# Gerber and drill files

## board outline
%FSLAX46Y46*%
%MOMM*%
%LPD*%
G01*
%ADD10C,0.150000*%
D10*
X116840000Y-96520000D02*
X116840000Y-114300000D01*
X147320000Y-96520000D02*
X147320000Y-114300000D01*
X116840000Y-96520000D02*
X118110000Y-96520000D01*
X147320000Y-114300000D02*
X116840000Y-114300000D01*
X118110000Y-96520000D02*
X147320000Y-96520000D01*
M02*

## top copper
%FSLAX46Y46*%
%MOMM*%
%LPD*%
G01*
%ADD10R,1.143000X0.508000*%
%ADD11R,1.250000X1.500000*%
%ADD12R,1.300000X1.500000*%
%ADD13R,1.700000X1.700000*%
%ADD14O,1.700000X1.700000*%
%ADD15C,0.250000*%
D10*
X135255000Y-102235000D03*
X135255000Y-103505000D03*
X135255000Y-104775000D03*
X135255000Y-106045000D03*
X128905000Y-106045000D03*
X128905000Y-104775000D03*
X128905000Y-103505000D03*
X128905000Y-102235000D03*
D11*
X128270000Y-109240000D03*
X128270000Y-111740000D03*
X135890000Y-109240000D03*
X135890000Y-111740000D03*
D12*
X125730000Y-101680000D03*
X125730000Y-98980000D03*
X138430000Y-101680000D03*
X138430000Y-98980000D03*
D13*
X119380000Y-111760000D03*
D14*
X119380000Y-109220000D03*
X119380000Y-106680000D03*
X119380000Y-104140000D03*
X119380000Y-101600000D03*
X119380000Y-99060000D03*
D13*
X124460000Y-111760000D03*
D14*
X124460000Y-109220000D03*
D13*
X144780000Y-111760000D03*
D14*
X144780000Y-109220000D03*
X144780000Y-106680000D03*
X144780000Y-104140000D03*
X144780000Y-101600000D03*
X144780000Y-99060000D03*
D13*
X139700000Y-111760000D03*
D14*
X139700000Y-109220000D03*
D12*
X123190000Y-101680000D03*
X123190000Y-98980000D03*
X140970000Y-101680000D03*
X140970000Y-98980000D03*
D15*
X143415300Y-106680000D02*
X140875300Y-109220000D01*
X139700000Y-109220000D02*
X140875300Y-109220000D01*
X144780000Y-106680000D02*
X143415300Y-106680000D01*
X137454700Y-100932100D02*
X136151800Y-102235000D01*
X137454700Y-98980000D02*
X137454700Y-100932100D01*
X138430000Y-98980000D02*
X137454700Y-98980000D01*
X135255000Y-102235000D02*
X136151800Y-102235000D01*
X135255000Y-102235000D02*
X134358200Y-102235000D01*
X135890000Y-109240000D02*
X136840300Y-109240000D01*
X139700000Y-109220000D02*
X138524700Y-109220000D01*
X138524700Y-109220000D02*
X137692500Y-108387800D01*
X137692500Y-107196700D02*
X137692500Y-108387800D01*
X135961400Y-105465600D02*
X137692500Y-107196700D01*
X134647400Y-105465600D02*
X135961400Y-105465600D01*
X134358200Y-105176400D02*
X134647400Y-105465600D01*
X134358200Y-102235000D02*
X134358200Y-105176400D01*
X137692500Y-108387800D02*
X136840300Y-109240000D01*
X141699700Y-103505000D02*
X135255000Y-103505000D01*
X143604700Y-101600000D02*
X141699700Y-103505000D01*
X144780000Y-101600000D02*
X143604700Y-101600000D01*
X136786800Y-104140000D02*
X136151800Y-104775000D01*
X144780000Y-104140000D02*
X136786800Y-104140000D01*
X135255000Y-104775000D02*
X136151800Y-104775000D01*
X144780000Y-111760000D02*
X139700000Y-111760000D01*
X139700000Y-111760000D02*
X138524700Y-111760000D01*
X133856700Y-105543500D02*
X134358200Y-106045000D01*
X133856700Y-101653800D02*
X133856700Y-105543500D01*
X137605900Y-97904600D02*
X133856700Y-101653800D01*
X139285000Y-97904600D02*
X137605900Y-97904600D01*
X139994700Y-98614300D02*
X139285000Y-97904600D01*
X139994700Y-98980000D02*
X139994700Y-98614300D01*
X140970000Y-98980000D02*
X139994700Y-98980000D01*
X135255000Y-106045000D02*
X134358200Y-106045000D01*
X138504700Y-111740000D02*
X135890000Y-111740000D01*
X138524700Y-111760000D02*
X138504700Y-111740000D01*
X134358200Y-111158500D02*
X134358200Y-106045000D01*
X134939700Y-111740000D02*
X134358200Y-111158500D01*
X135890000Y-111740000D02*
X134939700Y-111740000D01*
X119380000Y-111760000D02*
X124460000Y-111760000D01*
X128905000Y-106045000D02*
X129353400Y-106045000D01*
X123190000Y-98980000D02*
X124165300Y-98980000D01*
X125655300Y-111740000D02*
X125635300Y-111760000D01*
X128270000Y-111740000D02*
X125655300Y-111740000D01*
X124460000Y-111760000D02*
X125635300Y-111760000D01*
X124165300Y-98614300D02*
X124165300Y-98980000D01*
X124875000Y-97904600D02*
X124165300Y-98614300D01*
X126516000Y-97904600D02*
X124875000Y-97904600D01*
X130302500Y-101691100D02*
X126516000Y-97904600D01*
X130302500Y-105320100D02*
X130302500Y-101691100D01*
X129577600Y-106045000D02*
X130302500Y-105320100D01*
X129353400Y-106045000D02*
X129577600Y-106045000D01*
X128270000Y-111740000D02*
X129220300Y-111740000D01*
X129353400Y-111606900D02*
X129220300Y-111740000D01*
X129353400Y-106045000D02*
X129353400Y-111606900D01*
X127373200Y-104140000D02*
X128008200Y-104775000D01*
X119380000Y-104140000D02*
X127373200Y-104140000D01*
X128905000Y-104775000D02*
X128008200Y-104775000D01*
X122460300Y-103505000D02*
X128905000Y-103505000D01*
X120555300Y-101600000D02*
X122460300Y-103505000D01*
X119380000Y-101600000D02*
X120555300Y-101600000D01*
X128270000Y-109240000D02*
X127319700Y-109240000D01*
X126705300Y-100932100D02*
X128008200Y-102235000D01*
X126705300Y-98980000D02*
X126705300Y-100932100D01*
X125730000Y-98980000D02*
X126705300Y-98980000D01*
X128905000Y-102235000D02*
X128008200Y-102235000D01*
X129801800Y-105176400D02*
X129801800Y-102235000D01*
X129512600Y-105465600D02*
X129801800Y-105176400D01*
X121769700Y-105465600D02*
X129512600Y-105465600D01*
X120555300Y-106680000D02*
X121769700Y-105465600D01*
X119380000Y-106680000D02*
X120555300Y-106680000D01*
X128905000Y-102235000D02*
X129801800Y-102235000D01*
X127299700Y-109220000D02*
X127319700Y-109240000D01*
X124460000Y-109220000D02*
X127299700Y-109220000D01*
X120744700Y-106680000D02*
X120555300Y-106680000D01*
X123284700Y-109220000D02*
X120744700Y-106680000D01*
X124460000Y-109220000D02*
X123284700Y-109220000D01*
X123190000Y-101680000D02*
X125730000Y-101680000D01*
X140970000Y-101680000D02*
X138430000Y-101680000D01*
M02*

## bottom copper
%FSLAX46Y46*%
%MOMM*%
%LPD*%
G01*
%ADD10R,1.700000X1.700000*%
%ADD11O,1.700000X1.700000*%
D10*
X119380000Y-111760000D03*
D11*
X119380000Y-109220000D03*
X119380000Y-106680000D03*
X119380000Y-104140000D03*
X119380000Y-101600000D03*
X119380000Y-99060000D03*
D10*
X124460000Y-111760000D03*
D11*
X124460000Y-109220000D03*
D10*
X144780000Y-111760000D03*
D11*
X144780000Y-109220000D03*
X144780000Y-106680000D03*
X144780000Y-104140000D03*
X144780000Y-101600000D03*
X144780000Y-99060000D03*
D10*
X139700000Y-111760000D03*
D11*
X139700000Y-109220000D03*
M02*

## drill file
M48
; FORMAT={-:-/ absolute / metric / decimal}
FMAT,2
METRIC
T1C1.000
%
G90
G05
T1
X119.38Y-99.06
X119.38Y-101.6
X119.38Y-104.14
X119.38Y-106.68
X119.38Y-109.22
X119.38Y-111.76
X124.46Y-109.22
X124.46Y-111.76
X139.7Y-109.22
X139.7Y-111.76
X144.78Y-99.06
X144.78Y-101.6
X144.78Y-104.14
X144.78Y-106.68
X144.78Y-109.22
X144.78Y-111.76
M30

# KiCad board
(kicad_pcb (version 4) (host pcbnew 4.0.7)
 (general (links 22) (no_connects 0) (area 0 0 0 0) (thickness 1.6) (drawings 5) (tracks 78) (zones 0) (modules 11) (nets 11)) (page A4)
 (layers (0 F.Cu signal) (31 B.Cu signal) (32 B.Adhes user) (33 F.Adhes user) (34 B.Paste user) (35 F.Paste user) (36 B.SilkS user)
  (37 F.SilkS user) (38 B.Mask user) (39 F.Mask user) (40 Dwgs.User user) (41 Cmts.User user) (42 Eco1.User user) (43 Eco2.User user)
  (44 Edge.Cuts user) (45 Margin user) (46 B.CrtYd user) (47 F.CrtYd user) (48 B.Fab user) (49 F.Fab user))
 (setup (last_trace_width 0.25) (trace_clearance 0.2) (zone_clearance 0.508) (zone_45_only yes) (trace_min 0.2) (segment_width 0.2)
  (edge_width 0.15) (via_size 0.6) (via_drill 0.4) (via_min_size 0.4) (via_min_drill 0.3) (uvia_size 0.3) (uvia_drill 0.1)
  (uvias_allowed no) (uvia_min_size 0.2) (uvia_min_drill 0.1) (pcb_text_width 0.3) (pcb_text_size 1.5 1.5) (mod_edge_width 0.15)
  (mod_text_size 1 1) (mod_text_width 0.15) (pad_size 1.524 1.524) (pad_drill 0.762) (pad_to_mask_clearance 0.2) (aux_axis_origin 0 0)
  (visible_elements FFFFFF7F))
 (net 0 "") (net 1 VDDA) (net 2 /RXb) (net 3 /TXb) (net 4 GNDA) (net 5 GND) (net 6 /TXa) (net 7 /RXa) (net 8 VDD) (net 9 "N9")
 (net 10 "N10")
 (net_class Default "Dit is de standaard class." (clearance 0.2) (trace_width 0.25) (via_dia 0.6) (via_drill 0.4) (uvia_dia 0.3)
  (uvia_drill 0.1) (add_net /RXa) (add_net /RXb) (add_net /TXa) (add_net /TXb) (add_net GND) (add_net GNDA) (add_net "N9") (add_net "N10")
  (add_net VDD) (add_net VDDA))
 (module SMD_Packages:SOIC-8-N (layer F.Cu) (at 132.08 104.14 270)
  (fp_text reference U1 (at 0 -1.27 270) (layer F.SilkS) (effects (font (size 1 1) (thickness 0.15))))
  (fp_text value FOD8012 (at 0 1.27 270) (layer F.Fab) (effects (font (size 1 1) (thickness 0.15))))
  (pad 8 smd rect (at -1.905 -3.175 270) (size 0.508 1.143) (layers F.Cu F.Paste F.Mask) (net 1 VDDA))
  (pad 7 smd rect (at -0.635 -3.175 270) (size 0.508 1.143) (layers F.Cu F.Paste F.Mask) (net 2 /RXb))
  (pad 6 smd rect (at 0.635 -3.175 270) (size 0.508 1.143) (layers F.Cu F.Paste F.Mask) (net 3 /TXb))
  (pad 5 smd rect (at 1.905 -3.175 270) (size 0.508 1.143) (layers F.Cu F.Paste F.Mask) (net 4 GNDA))
  (pad 4 smd rect (at 1.905 3.175 270) (size 0.508 1.143) (layers F.Cu F.Paste F.Mask) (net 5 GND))
  (pad 3 smd rect (at 0.635 3.175 270) (size 0.508 1.143) (layers F.Cu F.Paste F.Mask) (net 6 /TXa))
  (pad 2 smd rect (at -0.635 3.175 270) (size 0.508 1.143) (layers F.Cu F.Paste F.Mask) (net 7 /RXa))
  (pad 1 smd rect (at -1.905 3.175 270) (size 0.508 1.143) (layers F.Cu F.Paste F.Mask) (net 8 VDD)))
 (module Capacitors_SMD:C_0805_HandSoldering (layer F.Cu) (at 128.27 110.49 270)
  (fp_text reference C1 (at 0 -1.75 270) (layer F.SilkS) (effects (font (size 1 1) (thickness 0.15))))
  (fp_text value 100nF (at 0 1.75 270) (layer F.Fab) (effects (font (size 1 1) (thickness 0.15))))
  (pad 1 smd rect (at -1.25 0 270) (size 1.5 1.25) (layers F.Cu F.Paste F.Mask) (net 8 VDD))
  (pad 2 smd rect (at 1.25 0 270) (size 1.5 1.25) (layers F.Cu F.Paste F.Mask) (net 5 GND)))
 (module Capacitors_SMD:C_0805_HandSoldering (layer F.Cu) (at 135.89 110.49 270)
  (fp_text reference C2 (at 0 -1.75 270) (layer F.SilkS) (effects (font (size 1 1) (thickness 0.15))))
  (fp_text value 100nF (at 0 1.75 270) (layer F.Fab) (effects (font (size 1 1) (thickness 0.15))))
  (pad 1 smd rect (at -1.25 0 270) (size 1.5 1.25) (layers F.Cu F.Paste F.Mask) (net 1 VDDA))
  (pad 2 smd rect (at 1.25 0 270) (size 1.5 1.25) (layers F.Cu F.Paste F.Mask) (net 4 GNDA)))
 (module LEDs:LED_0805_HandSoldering (layer F.Cu) (at 125.73 100.33 90)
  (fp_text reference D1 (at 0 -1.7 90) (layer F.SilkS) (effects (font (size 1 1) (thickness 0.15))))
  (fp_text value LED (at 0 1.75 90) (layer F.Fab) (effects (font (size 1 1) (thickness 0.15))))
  (pad 1 smd rect (at -1.35 0 90) (size 1.5 1.3) (layers F.Cu F.Paste F.Mask) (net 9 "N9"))
  (pad 2 smd rect (at 1.35 0 90) (size 1.5 1.3) (layers F.Cu F.Paste F.Mask) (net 8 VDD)))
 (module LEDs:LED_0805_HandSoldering (layer F.Cu) (at 138.43 100.33 90)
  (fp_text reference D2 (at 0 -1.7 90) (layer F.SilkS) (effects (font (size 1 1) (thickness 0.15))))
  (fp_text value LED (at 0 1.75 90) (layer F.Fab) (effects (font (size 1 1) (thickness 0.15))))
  (pad 1 smd rect (at -1.35 0 90) (size 1.5 1.3) (layers F.Cu F.Paste F.Mask) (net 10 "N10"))
  (pad 2 smd rect (at 1.35 0 90) (size 1.5 1.3) (layers F.Cu F.Paste F.Mask) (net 1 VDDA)))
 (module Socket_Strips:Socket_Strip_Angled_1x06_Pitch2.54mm (layer B.Cu) (at 119.38 111.76)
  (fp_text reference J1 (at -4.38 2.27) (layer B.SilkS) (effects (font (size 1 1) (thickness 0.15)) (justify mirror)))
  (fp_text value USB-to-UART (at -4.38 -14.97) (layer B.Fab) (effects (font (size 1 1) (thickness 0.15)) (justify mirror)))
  (pad 1 thru_hole rect (at 0 0) (size 1.7 1.7) (drill 1) (layers *.Cu *.Mask) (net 5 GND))
  (pad 2 thru_hole oval (at 0 -2.54) (size 1.7 1.7) (drill 1) (layers *.Cu *.Mask))
  (pad 3 thru_hole oval (at 0 -5.08) (size 1.7 1.7) (drill 1) (layers *.Cu *.Mask) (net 8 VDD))
  (pad 4 thru_hole oval (at 0 -7.62) (size 1.7 1.7) (drill 1) (layers *.Cu *.Mask) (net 6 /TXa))
  (pad 5 thru_hole oval (at 0 -10.16) (size 1.7 1.7) (drill 1) (layers *.Cu *.Mask) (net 7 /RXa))
  (pad 6 thru_hole oval (at 0 -12.7) (size 1.7 1.7) (drill 1) (layers *.Cu *.Mask)))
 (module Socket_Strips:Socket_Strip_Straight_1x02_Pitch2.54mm (layer F.Cu) (at 124.46 111.76 180)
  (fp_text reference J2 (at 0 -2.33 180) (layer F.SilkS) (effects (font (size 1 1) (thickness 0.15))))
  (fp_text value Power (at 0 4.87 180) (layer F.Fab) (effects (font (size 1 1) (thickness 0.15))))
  (pad 1 thru_hole rect (at 0 0 180) (size 1.7 1.7) (drill 1) (layers *.Cu *.Mask) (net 5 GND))
  (pad 2 thru_hole oval (at 0 2.54 180) (size 1.7 1.7) (drill 1) (layers *.Cu *.Mask) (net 8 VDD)))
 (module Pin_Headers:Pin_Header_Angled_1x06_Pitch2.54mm (layer B.Cu) (at 144.78 111.76)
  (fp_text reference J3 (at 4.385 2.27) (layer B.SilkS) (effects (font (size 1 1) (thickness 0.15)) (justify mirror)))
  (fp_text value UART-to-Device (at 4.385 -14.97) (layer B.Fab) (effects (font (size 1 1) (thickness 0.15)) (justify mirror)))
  (pad 1 thru_hole rect (at 0 0) (size 1.7 1.7) (drill 1) (layers *.Cu *.Mask) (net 4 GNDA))
  (pad 2 thru_hole oval (at 0 -2.54) (size 1.7 1.7) (drill 1) (layers *.Cu *.Mask))
  (pad 3 thru_hole oval (at 0 -5.08) (size 1.7 1.7) (drill 1) (layers *.Cu *.Mask) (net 1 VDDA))
  (pad 4 thru_hole oval (at 0 -7.62) (size 1.7 1.7) (drill 1) (layers *.Cu *.Mask) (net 3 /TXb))
  (pad 5 thru_hole oval (at 0 -10.16) (size 1.7 1.7) (drill 1) (layers *.Cu *.Mask) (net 2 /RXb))
  (pad 6 thru_hole oval (at 0 -12.7) (size 1.7 1.7) (drill 1) (layers *.Cu *.Mask)))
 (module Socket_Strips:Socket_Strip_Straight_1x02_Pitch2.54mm (layer F.Cu) (at 139.7 111.76 180)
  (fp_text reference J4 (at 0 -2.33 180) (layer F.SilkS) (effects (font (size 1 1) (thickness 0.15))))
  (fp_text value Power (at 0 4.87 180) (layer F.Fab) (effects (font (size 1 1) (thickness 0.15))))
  (pad 1 thru_hole rect (at 0 0 180) (size 1.7 1.7) (drill 1) (layers *.Cu *.Mask) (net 4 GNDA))
  (pad 2 thru_hole oval (at 0 2.54 180) (size 1.7 1.7) (drill 1) (layers *.Cu *.Mask) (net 1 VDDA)))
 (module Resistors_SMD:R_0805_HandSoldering (layer F.Cu) (at 123.19 100.33 90)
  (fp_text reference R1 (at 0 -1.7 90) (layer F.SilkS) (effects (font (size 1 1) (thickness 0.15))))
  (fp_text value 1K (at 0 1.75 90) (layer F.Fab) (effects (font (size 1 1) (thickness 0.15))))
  (pad 1 smd rect (at -1.35 0 90) (size 1.5 1.3) (layers F.Cu F.Paste F.Mask) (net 9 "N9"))
  (pad 2 smd rect (at 1.35 0 90) (size 1.5 1.3) (layers F.Cu F.Paste F.Mask) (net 5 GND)))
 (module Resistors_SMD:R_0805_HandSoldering (layer F.Cu) (at 140.97 100.33 90)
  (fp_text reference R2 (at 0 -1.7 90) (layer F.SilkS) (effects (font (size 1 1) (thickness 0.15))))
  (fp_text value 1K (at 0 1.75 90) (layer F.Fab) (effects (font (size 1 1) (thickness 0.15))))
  (pad 1 smd rect (at -1.35 0 90) (size 1.5 1.3) (layers F.Cu F.Paste F.Mask) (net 10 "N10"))
  (pad 2 smd rect (at 1.35 0 90) (size 1.5 1.3) (layers F.Cu F.Paste F.Mask) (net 4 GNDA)))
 (gr_line (start 116.84 96.52) (end 116.84 114.3) (angle 90) (layer Edge.Cuts) (width 0.15))
 (gr_line (start 147.32 96.52) (end 147.32 114.3) (angle 90) (layer Edge.Cuts) (width 0.15))
 (gr_line (start 116.84 96.52) (end 118.11 96.52) (angle 90) (layer Edge.Cuts) (width 0.15))
 (gr_line (start 147.32 114.3) (end 116.84 114.3) (angle 90) (layer Edge.Cuts) (width 0.15))
 (gr_line (start 118.11 96.52) (end 147.32 96.52) (angle 90) (layer Edge.Cuts) (width 0.15))
 (segment (start 143.4153 106.68) (end 140.8753 109.22) (width 0.25) (layer F.Cu) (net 1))
 (segment (start 139.7 109.22) (end 140.8753 109.22) (width 0.25) (layer F.Cu) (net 1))
 (segment (start 144.78 106.68) (end 143.4153 106.68) (width 0.25) (layer F.Cu) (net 1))
 (segment (start 137.4547 100.9321) (end 136.1518 102.235) (width 0.25) (layer F.Cu) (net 1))
 (segment (start 137.4547 98.98) (end 137.4547 100.9321) (width 0.25) (layer F.Cu) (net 1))
 (segment (start 138.43 98.98) (end 137.4547 98.98) (width 0.25) (layer F.Cu) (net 1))
 (segment (start 135.255 102.235) (end 136.1518 102.235) (width 0.25) (layer F.Cu) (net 1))
 (segment (start 135.255 102.235) (end 134.3582 102.235) (width 0.25) (layer F.Cu) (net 1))
 (segment (start 135.89 109.24) (end 136.8403 109.24) (width 0.25) (layer F.Cu) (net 1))
 (segment (start 139.7 109.22) (end 138.5247 109.22) (width 0.25) (layer F.Cu) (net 1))
 (segment (start 138.5247 109.22) (end 137.6925 108.3878) (width 0.25) (layer F.Cu) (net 1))
 (segment (start 137.6925 107.1967) (end 137.6925 108.3878) (width 0.25) (layer F.Cu) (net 1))
 (segment (start 135.9614 105.4656) (end 137.6925 107.1967) (width 0.25) (layer F.Cu) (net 1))
 (segment (start 134.6474 105.4656) (end 135.9614 105.4656) (width 0.25) (layer F.Cu) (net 1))
 (segment (start 134.3582 105.1764) (end 134.6474 105.4656) (width 0.25) (layer F.Cu) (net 1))
 (segment (start 134.3582 102.235) (end 134.3582 105.1764) (width 0.25) (layer F.Cu) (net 1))
 (segment (start 137.6925 108.3878) (end 136.8403 109.24) (width 0.25) (layer F.Cu) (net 1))
 (segment (start 141.6997 103.505) (end 135.255 103.505) (width 0.25) (layer F.Cu) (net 2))
 (segment (start 143.6047 101.6) (end 141.6997 103.505) (width 0.25) (layer F.Cu) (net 2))
 (segment (start 144.78 101.6) (end 143.6047 101.6) (width 0.25) (layer F.Cu) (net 2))
 (segment (start 136.7868 104.14) (end 136.1518 104.775) (width 0.25) (layer F.Cu) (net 3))
 (segment (start 144.78 104.14) (end 136.7868 104.14) (width 0.25) (layer F.Cu) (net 3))
 (segment (start 135.255 104.775) (end 136.1518 104.775) (width 0.25) (layer F.Cu) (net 3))
 (segment (start 144.78 111.76) (end 139.7 111.76) (width 0.25) (layer F.Cu) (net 4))
 (segment (start 139.7 111.76) (end 138.5247 111.76) (width 0.25) (layer F.Cu) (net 4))
 (segment (start 133.8567 105.5435) (end 134.3582 106.045) (width 0.25) (layer F.Cu) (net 4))
 (segment (start 133.8567 101.6538) (end 133.8567 105.5435) (width 0.25) (layer F.Cu) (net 4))
 (segment (start 137.6059 97.9046) (end 133.8567 101.6538) (width 0.25) (layer F.Cu) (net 4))
 (segment (start 139.285 97.9046) (end 137.6059 97.9046) (width 0.25) (layer F.Cu) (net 4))
 (segment (start 139.9947 98.6143) (end 139.285 97.9046) (width 0.25) (layer F.Cu) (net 4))
 (segment (start 139.9947 98.98) (end 139.9947 98.6143) (width 0.25) (layer F.Cu) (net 4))
 (segment (start 140.97 98.98) (end 139.9947 98.98) (width 0.25) (layer F.Cu) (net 4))
 (segment (start 135.255 106.045) (end 134.3582 106.045) (width 0.25) (layer F.Cu) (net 4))
 (segment (start 138.5047 111.74) (end 135.89 111.74) (width 0.25) (layer F.Cu) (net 4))
 (segment (start 138.5247 111.76) (end 138.5047 111.74) (width 0.25) (layer F.Cu) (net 4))
 (segment (start 134.3582 111.1585) (end 134.3582 106.045) (width 0.25) (layer F.Cu) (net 4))
 (segment (start 134.9397 111.74) (end 134.3582 111.1585) (width 0.25) (layer F.Cu) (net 4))
 (segment (start 135.89 111.74) (end 134.9397 111.74) (width 0.25) (layer F.Cu) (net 4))
 (segment (start 119.38 111.76) (end 124.46 111.76) (width 0.25) (layer F.Cu) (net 5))
 (segment (start 128.905 106.045) (end 129.3534 106.045) (width 0.25) (layer F.Cu) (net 5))
 (segment (start 123.19 98.98) (end 124.1653 98.98) (width 0.25) (layer F.Cu) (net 5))
 (segment (start 125.6553 111.74) (end 125.6353 111.76) (width 0.25) (layer F.Cu) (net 5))
 (segment (start 128.27 111.74) (end 125.6553 111.74) (width 0.25) (layer F.Cu) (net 5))
 (segment (start 124.46 111.76) (end 125.6353 111.76) (width 0.25) (layer F.Cu) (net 5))
 (segment (start 124.1653 98.6143) (end 124.1653 98.98) (width 0.25) (layer F.Cu) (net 5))
 (segment (start 124.875 97.9046) (end 124.1653 98.6143) (width 0.25) (layer F.Cu) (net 5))
 (segment (start 126.516 97.9046) (end 124.875 97.9046) (width 0.25) (layer F.Cu) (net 5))
 (segment (start 130.3025 101.6911) (end 126.516 97.9046) (width 0.25) (layer F.Cu) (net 5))
 (segment (start 130.3025 105.3201) (end 130.3025 101.6911) (width 0.25) (layer F.Cu) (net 5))
 (segment (start 129.5776 106.045) (end 130.3025 105.3201) (width 0.25) (layer F.Cu) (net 5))
 (segment (start 129.3534 106.045) (end 129.5776 106.045) (width 0.25) (layer F.Cu) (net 5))
 (segment (start 128.27 111.74) (end 129.2203 111.74) (width 0.25) (layer F.Cu) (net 5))
 (segment (start 129.3534 111.6069) (end 129.2203 111.74) (width 0.25) (layer F.Cu) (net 5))
 (segment (start 129.3534 106.045) (end 129.3534 111.6069) (width 0.25) (layer F.Cu) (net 5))
 (segment (start 127.3732 104.14) (end 128.0082 104.775) (width 0.25) (layer F.Cu) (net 6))
 (segment (start 119.38 104.14) (end 127.3732 104.14) (width 0.25) (layer F.Cu) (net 6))
 (segment (start 128.905 104.775) (end 128.0082 104.775) (width 0.25) (layer F.Cu) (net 6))
 (segment (start 122.4603 103.505) (end 128.905 103.505) (width 0.25) (layer F.Cu) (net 7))
 (segment (start 120.5553 101.6) (end 122.4603 103.505) (width 0.25) (layer F.Cu) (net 7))
 (segment (start 119.38 101.6) (end 120.5553 101.6) (width 0.25) (layer F.Cu) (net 7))
 (segment (start 128.27 109.24) (end 127.3197 109.24) (width 0.25) (layer F.Cu) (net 8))
 (segment (start 126.7053 100.9321) (end 128.0082 102.235) (width 0.25) (layer F.Cu) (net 8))
 (segment (start 126.7053 98.98) (end 126.7053 100.9321) (width 0.25) (layer F.Cu) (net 8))
 (segment (start 125.73 98.98) (end 126.7053 98.98) (width 0.25) (layer F.Cu) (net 8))
 (segment (start 128.905 102.235) (end 128.0082 102.235) (width 0.25) (layer F.Cu) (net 8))
 (segment (start 129.8018 105.1764) (end 129.8018 102.235) (width 0.25) (layer F.Cu) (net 8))
 (segment (start 129.5126 105.4656) (end 129.8018 105.1764) (width 0.25) (layer F.Cu) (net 8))
 (segment (start 121.7697 105.4656) (end 129.5126 105.4656) (width 0.25) (layer F.Cu) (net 8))
 (segment (start 120.5553 106.68) (end 121.7697 105.4656) (width 0.25) (layer F.Cu) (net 8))
 (segment (start 119.38 106.68) (end 120.5553 106.68) (width 0.25) (layer F.Cu) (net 8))
 (segment (start 128.905 102.235) (end 129.8018 102.235) (width 0.25) (layer F.Cu) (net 8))
 (segment (start 127.2997 109.22) (end 127.3197 109.24) (width 0.25) (layer F.Cu) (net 8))
 (segment (start 124.46 109.22) (end 127.2997 109.22) (width 0.25) (layer F.Cu) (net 8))
 (segment (start 120.7447 106.68) (end 120.5553 106.68) (width 0.25) (layer F.Cu) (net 8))
 (segment (start 123.2847 109.22) (end 120.7447 106.68) (width 0.25) (layer F.Cu) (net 8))
 (segment (start 124.46 109.22) (end 123.2847 109.22) (width 0.25) (layer F.Cu) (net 8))
 (segment (start 123.19 101.68) (end 125.73 101.68) (width 0.25) (layer F.Cu) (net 9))
 (segment (start 140.97 101.68) (end 138.43 101.68) (width 0.25) (layer F.Cu) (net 10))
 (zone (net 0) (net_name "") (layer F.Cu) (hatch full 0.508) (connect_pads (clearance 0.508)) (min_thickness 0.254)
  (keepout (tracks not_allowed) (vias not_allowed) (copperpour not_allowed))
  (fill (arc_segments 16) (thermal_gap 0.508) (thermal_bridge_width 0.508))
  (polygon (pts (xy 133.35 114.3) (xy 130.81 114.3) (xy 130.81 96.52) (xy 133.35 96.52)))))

